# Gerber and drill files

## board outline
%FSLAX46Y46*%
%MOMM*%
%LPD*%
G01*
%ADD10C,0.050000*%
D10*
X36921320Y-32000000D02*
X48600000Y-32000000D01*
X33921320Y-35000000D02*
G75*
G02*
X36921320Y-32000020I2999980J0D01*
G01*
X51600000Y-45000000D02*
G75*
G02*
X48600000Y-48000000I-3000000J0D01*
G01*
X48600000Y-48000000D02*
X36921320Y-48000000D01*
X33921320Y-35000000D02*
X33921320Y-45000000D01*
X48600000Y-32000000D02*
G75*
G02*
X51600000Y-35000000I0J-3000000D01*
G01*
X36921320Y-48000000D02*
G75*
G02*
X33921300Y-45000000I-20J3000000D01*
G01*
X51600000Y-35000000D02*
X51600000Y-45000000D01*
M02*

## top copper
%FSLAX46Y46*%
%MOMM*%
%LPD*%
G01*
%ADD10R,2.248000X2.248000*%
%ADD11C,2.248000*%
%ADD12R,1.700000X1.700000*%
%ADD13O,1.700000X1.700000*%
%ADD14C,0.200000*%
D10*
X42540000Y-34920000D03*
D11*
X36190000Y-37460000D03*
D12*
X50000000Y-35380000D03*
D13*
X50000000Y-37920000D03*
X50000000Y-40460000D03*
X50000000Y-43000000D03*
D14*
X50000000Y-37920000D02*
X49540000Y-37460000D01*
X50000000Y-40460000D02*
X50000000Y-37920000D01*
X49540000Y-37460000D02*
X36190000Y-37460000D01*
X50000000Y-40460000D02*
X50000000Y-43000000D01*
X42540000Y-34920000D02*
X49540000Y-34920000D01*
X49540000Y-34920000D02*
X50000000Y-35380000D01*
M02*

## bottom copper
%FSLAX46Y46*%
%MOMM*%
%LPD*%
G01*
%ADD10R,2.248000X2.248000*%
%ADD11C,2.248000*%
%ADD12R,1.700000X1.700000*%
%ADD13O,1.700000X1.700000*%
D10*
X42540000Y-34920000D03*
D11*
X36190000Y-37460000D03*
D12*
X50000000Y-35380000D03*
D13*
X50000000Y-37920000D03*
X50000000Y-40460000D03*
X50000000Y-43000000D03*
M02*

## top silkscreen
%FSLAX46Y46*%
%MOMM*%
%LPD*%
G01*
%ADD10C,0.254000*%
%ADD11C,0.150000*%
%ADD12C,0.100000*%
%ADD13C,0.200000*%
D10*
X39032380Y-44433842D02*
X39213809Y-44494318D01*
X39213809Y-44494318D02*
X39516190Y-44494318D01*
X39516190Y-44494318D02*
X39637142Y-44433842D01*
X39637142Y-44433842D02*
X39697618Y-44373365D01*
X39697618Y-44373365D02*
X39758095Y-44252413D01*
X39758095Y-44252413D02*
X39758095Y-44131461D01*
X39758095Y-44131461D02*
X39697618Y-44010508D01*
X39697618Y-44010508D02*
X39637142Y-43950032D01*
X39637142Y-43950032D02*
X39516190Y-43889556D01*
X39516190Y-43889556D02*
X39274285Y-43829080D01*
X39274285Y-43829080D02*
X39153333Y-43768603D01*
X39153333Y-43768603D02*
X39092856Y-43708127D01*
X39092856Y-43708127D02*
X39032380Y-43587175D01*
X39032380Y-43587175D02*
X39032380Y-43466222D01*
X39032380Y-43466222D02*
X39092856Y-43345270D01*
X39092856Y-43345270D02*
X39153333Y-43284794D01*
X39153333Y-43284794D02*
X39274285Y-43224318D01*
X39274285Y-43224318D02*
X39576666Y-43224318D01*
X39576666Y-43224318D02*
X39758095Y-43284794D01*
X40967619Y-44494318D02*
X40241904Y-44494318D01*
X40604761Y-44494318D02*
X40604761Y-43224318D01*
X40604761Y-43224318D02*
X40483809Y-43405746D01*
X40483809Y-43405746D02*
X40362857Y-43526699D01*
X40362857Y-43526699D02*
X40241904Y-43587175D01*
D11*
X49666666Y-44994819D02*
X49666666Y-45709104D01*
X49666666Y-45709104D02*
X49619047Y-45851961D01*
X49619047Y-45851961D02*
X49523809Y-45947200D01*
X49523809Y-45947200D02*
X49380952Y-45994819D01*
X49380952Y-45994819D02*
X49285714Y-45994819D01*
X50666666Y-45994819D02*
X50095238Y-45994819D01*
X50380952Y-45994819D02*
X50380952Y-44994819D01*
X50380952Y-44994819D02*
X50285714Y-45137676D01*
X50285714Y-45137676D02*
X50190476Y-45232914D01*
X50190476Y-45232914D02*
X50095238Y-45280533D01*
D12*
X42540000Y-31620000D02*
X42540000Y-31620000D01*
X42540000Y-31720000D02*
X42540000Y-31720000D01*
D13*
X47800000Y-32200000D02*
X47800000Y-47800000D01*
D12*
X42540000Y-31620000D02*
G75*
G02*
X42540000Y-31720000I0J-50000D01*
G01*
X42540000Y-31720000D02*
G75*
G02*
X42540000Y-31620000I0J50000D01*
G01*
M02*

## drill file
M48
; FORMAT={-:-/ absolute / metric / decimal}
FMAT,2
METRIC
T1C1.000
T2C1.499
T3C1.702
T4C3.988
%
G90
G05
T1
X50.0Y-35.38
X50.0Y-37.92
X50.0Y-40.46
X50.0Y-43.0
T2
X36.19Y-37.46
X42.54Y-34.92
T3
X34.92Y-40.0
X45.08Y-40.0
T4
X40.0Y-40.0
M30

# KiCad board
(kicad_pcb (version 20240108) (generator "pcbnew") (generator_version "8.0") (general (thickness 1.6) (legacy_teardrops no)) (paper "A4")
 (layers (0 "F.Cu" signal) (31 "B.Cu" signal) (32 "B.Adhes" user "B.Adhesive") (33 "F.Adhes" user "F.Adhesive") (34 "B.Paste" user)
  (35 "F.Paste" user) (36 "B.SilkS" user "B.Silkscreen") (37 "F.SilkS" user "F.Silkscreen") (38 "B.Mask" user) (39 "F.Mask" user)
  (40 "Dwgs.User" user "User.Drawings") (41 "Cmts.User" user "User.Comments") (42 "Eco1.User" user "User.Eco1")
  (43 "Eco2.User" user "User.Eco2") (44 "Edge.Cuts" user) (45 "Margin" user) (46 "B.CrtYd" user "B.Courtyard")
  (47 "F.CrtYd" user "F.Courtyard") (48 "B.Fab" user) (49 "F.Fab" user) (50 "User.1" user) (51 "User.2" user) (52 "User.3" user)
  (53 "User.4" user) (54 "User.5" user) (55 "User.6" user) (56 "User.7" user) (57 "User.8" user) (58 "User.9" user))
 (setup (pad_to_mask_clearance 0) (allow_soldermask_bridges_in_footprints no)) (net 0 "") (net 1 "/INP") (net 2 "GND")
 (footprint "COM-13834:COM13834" (layer "F.Cu") (at 42.54 34.92)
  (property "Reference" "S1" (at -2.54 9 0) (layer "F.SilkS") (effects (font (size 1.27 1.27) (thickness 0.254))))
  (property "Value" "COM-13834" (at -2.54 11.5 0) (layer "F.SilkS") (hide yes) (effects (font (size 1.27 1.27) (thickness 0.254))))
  (fp_line (start 0 -3.3) (end 0 -3.3) (stroke (width 0.1) (type solid)) (layer "F.SilkS"))
  (fp_line (start 0 -3.2) (end 0 -3.2) (stroke (width 0.1) (type solid)) (layer "F.SilkS"))
  (fp_line (start 5.26 -2.72) (end 5.26 12.88) (stroke (width 0.2) (type solid)) (layer "F.SilkS"))
  (fp_arc (start 0 -3.3) (mid 0.05 -3.25) (end 0 -3.2) (stroke (width 0.1) (type solid)) (layer "F.SilkS"))
  (fp_arc (start 0 -3.2) (mid -0.05 -3.25) (end 0 -3.3) (stroke (width 0.1) (type solid)) (layer "F.SilkS"))
  (pad "" np_thru_hole circle (at -7.62 5.08) (size 1.7018 1.7018) (drill 1.7018) (layers "*.Cu" "*.Mask"))
  (pad "" np_thru_hole circle (at -2.54 5.08) (size 3.9878 3.9878) (drill 3.9878) (layers "*.Cu" "*.Mask"))
  (pad "" np_thru_hole circle (at 2.54 5.08) (size 1.7018 1.7018) (drill 1.7018) (layers "*.Cu" "*.Mask"))
  (pad "1" thru_hole rect (at 0 0) (size 2.248 2.248) (drill 1.4986) (layers "*.Cu" "*.Mask") (remove_unused_layers no) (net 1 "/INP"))
  (pad "2" thru_hole circle (at -6.35 2.54) (size 2.248 2.248) (drill 1.4986) (layers "*.Cu" "*.Mask") (remove_unused_layers no)
   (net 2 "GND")))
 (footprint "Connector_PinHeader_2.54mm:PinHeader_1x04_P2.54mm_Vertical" (layer "B.Cu") (at 50 35.38 180)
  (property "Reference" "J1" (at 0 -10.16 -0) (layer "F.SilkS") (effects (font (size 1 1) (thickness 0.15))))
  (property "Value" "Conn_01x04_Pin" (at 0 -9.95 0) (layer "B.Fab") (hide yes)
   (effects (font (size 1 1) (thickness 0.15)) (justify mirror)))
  (pad "1" thru_hole rect (at 0 0 180) (size 1.7 1.7) (drill 1) (layers "*.Cu" "*.Mask") (remove_unused_layers no) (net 1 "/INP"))
  (pad "2" thru_hole oval (at 0 -2.54 180) (size 1.7 1.7) (drill 1) (layers "*.Cu" "*.Mask") (remove_unused_layers no) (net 2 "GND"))
  (pad "3" thru_hole oval (at 0 -5.08 180) (size 1.7 1.7) (drill 1) (layers "*.Cu" "*.Mask") (remove_unused_layers no) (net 2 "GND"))
  (pad "4" thru_hole oval (at 0 -7.62 180) (size 1.7 1.7) (drill 1) (layers "*.Cu" "*.Mask") (remove_unused_layers no) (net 2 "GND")))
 (gr_line (start 36.92132 32) (end 48.6 32) (stroke (width 0.05) (type default)) (layer "Edge.Cuts"))
 (gr_arc (start 33.92132 35) (mid 34.8 32.87868) (end 36.92132 32) (stroke (width 0.05) (type default)) (layer "Edge.Cuts"))
 (gr_arc (start 51.6 45) (mid 50.72132 47.12132) (end 48.6 48) (stroke (width 0.05) (type default)) (layer "Edge.Cuts"))
 (gr_line (start 48.6 48) (end 36.92132 48) (stroke (width 0.05) (type default)) (layer "Edge.Cuts"))
 (gr_line (start 33.92132 35) (end 33.92132 45) (stroke (width 0.05) (type default)) (layer "Edge.Cuts"))
 (gr_arc (start 48.6 32) (mid 50.72132 32.87868) (end 51.6 35) (stroke (width 0.05) (type default)) (layer "Edge.Cuts"))
 (gr_arc (start 36.92132 48) (mid 34.8 47.12132) (end 33.92132 45) (stroke (width 0.05) (type default)) (layer "Edge.Cuts"))
 (gr_line (start 51.6 35) (end 51.6 45) (stroke (width 0.05) (type default)) (layer "Edge.Cuts"))
 (segment (start 50 37.92) (end 49.54 37.46) (width 0.2) (layer "F.Cu") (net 2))
 (segment (start 50 40.46) (end 50 37.92) (width 0.2) (layer "F.Cu") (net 2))
 (segment (start 49.54 37.46) (end 36.19 37.46) (width 0.2) (layer "F.Cu") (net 2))
 (segment (start 50 40.46) (end 50 43) (width 0.2) (layer "F.Cu") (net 2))
 (segment (start 42.54 34.92) (end 49.54 34.92) (width 0.2) (layer "F.Cu") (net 1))
 (segment (start 49.54 34.92) (end 50 35.38) (width 0.2) (layer "F.Cu") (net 1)))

